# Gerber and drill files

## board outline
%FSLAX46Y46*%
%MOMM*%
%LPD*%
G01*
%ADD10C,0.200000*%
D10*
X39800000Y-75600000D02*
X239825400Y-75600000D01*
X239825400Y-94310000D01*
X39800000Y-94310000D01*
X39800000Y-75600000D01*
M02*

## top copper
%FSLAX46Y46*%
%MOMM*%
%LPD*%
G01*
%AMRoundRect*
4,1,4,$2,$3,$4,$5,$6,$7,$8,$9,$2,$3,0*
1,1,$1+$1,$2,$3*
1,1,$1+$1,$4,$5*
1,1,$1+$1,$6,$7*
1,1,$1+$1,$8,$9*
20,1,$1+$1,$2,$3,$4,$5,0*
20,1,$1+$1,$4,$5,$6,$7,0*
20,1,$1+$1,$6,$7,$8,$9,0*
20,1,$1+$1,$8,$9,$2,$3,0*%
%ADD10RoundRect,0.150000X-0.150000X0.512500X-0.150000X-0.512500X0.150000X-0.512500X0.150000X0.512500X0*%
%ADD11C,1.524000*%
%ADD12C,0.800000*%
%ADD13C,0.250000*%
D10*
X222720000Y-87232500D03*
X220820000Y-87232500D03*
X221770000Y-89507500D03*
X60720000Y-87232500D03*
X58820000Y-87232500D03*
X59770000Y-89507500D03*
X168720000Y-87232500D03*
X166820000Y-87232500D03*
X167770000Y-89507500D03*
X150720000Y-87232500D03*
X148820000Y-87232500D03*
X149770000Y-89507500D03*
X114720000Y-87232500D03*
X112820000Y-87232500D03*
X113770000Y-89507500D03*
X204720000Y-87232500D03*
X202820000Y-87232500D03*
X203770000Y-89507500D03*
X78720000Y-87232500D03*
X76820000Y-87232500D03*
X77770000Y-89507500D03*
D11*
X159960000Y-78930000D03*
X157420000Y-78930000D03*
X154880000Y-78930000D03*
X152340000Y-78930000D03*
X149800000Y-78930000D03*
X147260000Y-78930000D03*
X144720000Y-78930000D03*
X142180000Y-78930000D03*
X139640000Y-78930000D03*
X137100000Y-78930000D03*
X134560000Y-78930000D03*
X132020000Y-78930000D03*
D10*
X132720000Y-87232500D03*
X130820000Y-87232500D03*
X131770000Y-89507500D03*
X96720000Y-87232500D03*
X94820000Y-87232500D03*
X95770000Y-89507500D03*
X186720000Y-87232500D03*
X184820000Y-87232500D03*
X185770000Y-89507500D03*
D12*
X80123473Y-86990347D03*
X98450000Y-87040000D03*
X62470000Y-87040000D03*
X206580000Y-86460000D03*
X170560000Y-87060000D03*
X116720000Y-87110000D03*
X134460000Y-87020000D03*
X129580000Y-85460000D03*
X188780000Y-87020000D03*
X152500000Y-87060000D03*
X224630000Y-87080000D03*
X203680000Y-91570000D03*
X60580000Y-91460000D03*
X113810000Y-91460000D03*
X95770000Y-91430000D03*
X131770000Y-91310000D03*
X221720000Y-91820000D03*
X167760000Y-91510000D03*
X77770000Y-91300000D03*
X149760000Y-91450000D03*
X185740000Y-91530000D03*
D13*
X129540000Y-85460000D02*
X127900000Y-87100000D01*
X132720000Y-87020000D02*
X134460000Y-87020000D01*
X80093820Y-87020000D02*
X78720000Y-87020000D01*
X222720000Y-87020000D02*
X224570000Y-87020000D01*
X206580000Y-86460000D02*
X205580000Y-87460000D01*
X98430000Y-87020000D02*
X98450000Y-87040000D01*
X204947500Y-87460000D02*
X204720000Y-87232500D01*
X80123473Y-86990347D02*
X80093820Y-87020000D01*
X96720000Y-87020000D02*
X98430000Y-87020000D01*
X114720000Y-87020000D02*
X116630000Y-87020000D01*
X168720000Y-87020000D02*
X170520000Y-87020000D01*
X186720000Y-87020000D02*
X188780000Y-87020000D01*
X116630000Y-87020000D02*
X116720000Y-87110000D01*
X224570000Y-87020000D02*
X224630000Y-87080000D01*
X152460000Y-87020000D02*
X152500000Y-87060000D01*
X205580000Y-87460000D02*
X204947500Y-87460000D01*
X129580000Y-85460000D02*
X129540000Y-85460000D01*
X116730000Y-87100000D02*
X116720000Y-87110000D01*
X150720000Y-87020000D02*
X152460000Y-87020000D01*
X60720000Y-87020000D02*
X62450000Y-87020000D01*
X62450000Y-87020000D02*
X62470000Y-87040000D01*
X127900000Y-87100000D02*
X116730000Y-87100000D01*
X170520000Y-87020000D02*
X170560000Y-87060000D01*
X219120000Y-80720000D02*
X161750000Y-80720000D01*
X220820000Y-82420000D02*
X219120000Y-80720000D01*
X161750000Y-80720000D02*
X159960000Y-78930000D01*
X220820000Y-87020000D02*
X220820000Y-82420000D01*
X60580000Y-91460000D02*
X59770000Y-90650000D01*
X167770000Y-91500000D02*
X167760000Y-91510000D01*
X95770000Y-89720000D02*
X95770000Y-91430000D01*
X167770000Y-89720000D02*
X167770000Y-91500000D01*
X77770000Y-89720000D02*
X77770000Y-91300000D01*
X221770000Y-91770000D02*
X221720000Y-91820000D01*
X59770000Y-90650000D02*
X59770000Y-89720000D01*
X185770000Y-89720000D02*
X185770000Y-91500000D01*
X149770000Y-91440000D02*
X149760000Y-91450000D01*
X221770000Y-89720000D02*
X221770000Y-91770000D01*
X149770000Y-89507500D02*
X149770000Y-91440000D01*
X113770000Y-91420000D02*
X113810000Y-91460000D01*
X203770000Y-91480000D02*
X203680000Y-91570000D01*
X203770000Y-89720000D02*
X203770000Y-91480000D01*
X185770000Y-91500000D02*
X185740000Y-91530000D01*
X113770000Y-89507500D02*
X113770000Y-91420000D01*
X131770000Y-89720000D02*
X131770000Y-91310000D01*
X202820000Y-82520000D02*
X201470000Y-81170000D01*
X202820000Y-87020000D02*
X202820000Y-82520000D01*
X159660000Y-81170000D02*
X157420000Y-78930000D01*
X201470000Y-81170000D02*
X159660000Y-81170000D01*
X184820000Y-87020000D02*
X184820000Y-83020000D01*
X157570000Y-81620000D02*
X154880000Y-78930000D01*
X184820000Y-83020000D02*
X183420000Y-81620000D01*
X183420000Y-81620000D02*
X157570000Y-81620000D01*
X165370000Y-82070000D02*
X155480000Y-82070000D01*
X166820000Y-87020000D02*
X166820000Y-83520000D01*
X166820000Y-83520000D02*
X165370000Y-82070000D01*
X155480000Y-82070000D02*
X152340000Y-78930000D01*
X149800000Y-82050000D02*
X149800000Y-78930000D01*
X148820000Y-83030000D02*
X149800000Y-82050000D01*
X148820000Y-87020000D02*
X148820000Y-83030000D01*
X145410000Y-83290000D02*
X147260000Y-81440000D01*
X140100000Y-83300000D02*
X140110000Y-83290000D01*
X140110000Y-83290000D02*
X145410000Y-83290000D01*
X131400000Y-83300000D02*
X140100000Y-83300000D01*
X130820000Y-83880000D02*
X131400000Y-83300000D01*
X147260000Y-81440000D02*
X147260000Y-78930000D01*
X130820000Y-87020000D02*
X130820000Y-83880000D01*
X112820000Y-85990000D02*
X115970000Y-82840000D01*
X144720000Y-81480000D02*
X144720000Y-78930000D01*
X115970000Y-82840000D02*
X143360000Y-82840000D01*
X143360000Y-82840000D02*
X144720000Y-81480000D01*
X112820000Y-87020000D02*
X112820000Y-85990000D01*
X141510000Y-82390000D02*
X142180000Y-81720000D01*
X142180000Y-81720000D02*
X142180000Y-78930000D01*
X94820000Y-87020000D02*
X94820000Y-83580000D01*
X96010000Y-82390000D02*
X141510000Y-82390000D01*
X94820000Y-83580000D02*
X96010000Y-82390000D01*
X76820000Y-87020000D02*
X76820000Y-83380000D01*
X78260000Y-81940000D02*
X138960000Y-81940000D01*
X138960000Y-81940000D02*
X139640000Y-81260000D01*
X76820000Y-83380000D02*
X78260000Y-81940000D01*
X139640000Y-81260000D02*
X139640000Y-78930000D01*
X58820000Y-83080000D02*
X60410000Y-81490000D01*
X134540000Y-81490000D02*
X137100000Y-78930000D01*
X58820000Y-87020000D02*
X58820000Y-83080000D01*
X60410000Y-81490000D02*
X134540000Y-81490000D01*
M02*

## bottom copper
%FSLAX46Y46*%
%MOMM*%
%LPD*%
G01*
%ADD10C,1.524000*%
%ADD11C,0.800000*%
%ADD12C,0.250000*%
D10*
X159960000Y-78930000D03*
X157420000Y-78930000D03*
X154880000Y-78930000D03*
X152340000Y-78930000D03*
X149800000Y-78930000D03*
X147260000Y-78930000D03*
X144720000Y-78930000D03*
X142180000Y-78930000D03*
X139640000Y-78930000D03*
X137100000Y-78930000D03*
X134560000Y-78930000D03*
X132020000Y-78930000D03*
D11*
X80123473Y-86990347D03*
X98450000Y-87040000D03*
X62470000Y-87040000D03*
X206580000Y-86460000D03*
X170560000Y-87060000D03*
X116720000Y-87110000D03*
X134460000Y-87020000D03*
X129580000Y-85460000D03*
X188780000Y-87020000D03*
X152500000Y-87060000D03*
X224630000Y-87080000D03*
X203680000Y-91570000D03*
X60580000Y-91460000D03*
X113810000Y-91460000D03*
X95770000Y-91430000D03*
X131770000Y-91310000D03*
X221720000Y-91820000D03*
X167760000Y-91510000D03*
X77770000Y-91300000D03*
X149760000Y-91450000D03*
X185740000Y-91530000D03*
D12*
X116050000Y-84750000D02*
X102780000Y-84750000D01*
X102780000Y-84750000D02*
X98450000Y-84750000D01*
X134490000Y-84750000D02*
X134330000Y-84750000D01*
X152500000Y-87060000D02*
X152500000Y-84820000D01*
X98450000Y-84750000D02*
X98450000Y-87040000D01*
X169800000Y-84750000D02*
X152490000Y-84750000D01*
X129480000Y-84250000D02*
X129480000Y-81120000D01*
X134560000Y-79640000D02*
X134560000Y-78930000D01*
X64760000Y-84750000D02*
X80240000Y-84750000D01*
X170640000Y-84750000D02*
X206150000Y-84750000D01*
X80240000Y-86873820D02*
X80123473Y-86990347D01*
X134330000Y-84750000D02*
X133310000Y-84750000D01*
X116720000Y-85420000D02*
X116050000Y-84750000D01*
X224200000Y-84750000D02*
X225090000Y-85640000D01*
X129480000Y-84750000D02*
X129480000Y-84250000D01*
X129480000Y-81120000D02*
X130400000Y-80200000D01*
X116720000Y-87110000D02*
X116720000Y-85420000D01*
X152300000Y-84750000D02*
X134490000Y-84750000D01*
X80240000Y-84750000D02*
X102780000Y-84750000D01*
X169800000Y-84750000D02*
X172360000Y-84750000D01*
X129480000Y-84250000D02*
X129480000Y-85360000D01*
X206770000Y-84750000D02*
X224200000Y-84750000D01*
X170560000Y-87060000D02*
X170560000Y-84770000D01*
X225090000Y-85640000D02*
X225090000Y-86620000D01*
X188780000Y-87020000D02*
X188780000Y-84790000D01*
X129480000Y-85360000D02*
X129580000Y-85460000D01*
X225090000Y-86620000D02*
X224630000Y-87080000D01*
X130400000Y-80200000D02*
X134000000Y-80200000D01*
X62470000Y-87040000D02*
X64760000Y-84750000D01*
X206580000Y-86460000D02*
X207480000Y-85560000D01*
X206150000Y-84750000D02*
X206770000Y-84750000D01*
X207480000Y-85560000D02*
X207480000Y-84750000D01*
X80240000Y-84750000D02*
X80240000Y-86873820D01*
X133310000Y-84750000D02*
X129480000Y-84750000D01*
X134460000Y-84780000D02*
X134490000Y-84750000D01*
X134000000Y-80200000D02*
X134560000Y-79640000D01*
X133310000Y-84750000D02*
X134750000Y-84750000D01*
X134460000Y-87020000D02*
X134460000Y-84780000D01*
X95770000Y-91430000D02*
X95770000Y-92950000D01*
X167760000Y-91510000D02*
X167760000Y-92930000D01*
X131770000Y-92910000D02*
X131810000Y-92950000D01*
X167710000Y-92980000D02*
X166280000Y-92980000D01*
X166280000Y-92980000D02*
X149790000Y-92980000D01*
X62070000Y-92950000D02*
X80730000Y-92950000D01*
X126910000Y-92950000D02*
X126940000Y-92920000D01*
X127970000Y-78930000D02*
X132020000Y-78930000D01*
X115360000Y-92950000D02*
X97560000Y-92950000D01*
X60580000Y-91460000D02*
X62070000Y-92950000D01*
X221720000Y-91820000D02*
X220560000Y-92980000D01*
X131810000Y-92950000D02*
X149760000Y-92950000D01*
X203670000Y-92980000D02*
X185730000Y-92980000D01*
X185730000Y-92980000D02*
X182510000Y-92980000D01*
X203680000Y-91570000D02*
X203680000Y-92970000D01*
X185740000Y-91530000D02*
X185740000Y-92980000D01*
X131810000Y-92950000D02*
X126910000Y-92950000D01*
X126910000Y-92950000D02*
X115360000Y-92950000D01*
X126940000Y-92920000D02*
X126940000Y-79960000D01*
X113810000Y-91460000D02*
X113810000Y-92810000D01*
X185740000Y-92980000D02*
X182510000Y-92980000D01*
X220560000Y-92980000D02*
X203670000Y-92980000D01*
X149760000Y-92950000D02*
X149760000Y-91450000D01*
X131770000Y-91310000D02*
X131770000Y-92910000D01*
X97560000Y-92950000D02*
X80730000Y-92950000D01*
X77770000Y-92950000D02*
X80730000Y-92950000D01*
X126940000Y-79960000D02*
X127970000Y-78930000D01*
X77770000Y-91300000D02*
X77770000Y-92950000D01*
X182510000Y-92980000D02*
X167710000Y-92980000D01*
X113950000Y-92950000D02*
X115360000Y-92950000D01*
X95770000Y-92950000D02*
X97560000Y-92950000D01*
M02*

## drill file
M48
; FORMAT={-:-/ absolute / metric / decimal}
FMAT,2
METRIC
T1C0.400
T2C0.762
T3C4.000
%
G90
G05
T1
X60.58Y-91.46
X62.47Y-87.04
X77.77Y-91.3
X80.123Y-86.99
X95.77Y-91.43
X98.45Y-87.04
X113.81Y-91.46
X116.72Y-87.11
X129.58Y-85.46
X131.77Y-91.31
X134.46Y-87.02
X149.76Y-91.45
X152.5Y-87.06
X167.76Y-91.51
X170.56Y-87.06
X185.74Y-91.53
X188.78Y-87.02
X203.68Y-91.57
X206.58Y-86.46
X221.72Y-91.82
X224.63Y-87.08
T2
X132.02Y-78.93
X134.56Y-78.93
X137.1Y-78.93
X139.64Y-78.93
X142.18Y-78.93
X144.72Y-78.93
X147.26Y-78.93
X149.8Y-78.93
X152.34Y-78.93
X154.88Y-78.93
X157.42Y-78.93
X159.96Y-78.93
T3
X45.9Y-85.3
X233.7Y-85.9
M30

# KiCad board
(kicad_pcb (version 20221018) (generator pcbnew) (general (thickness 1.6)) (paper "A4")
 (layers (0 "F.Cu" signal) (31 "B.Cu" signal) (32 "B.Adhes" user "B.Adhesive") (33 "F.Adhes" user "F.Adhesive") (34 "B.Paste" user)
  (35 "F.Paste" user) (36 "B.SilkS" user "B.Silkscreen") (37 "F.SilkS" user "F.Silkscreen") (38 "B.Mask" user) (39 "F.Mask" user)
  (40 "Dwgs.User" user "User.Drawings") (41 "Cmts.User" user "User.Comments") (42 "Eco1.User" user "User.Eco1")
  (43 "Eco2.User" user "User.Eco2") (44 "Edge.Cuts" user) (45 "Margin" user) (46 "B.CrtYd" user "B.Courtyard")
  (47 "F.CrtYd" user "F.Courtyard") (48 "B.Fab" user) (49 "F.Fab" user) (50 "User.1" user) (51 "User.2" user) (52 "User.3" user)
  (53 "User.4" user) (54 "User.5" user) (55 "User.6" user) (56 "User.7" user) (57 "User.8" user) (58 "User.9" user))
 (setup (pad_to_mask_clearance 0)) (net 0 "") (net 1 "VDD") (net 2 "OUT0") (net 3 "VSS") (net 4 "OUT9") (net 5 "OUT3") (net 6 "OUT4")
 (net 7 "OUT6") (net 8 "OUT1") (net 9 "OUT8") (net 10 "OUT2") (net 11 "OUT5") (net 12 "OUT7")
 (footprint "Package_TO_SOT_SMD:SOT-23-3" (layer "F.Cu") (at 221.77 88.37 -90)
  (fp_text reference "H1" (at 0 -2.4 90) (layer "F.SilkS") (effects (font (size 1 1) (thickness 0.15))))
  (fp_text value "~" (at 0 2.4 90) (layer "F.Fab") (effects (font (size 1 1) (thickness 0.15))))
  (pad "1" smd roundrect (at -1.1375 -0.95 270) (size 1.325 0.6) (layers "F.Cu" "F.Paste" "F.Mask") (roundrect_rratio 0.25) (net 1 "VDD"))
  (pad "2" smd roundrect (at -1.1375 0.95 270) (size 1.325 0.6) (layers "F.Cu" "F.Paste" "F.Mask") (roundrect_rratio 0.25) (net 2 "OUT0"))
  (pad "3" smd roundrect (at 1.1375 0 270) (size 1.325 0.6) (layers "F.Cu" "F.Paste" "F.Mask") (roundrect_rratio 0.25) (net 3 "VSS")))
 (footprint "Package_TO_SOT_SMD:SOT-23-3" (layer "F.Cu") (at 59.77 88.37 -90)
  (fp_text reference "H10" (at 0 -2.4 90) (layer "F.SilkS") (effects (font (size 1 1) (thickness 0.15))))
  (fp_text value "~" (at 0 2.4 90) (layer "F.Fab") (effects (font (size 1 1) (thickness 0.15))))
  (pad "1" smd roundrect (at -1.1375 -0.95 270) (size 1.325 0.6) (layers "F.Cu" "F.Paste" "F.Mask") (roundrect_rratio 0.25) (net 1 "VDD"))
  (pad "2" smd roundrect (at -1.1375 0.95 270) (size 1.325 0.6) (layers "F.Cu" "F.Paste" "F.Mask") (roundrect_rratio 0.25) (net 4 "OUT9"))
  (pad "3" smd roundrect (at 1.1375 0 270) (size 1.325 0.6) (layers "F.Cu" "F.Paste" "F.Mask") (roundrect_rratio 0.25) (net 3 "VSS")))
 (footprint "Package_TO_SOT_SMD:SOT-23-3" (layer "F.Cu") (at 167.77 88.37 -90)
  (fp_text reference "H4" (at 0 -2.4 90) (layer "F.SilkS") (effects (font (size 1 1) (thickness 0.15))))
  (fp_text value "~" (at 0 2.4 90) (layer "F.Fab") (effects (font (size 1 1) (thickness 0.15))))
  (pad "1" smd roundrect (at -1.1375 -0.95 270) (size 1.325 0.6) (layers "F.Cu" "F.Paste" "F.Mask") (roundrect_rratio 0.25) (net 1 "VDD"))
  (pad "2" smd roundrect (at -1.1375 0.95 270) (size 1.325 0.6) (layers "F.Cu" "F.Paste" "F.Mask") (roundrect_rratio 0.25) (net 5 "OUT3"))
  (pad "3" smd roundrect (at 1.1375 0 270) (size 1.325 0.6) (layers "F.Cu" "F.Paste" "F.Mask") (roundrect_rratio 0.25) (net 3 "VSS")))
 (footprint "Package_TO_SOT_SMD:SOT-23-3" (layer "F.Cu") (at 149.77 88.37 -90)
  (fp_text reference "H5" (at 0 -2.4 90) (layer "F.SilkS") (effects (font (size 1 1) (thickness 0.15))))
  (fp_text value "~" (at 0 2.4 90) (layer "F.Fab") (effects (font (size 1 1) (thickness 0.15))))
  (pad "1" smd roundrect (at -1.1375 -0.95 270) (size 1.325 0.6) (layers "F.Cu" "F.Paste" "F.Mask") (roundrect_rratio 0.25) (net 1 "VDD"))
  (pad "2" smd roundrect (at -1.1375 0.95 270) (size 1.325 0.6) (layers "F.Cu" "F.Paste" "F.Mask") (roundrect_rratio 0.25) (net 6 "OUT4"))
  (pad "3" smd roundrect (at 1.1375 0 270) (size 1.325 0.6) (layers "F.Cu" "F.Paste" "F.Mask") (roundrect_rratio 0.25) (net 3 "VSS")))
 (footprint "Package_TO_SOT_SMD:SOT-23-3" (layer "F.Cu") (at 113.77 88.37 -90)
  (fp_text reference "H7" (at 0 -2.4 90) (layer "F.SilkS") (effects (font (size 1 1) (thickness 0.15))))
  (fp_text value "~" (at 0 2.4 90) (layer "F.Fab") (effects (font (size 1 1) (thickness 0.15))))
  (pad "1" smd roundrect (at -1.1375 -0.95 270) (size 1.325 0.6) (layers "F.Cu" "F.Paste" "F.Mask") (roundrect_rratio 0.25) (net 1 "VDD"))
  (pad "2" smd roundrect (at -1.1375 0.95 270) (size 1.325 0.6) (layers "F.Cu" "F.Paste" "F.Mask") (roundrect_rratio 0.25) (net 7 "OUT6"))
  (pad "3" smd roundrect (at 1.1375 0 270) (size 1.325 0.6) (layers "F.Cu" "F.Paste" "F.Mask") (roundrect_rratio 0.25) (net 3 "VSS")))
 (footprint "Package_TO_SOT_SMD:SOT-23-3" (layer "F.Cu") (at 203.77 88.37 -90)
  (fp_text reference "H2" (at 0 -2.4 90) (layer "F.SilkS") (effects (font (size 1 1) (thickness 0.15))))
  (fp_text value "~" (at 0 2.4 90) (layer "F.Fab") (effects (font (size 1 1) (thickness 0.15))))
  (pad "1" smd roundrect (at -1.1375 -0.95 270) (size 1.325 0.6) (layers "F.Cu" "F.Paste" "F.Mask") (roundrect_rratio 0.25) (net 1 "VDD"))
  (pad "2" smd roundrect (at -1.1375 0.95 270) (size 1.325 0.6) (layers "F.Cu" "F.Paste" "F.Mask") (roundrect_rratio 0.25) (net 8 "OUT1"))
  (pad "3" smd roundrect (at 1.1375 0 270) (size 1.325 0.6) (layers "F.Cu" "F.Paste" "F.Mask") (roundrect_rratio 0.25) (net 3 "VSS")))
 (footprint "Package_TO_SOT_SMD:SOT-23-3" (layer "F.Cu") (at 77.77 88.37 -90)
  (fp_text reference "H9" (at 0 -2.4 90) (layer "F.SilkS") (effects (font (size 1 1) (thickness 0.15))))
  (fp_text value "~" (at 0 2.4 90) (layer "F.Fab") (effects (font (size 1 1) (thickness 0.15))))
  (pad "1" smd roundrect (at -1.1375 -0.95 270) (size 1.325 0.6) (layers "F.Cu" "F.Paste" "F.Mask") (roundrect_rratio 0.25) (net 1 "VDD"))
  (pad "2" smd roundrect (at -1.1375 0.95 270) (size 1.325 0.6) (layers "F.Cu" "F.Paste" "F.Mask") (roundrect_rratio 0.25) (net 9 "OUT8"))
  (pad "3" smd roundrect (at 1.1375 0 270) (size 1.325 0.6) (layers "F.Cu" "F.Paste" "F.Mask") (roundrect_rratio 0.25) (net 3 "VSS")))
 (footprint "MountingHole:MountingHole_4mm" (layer "F.Cu") (at 233.7 85.9)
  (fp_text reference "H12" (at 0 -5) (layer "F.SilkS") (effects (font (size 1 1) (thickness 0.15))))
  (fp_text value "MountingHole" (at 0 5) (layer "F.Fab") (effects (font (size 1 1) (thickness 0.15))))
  (pad "" np_thru_hole circle (at 0 0) (size 4 4) (drill 4) (layers "*.Cu" "*.Mask")))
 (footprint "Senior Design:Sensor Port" (layer "F.Cu") (at 142.18 86.55 180)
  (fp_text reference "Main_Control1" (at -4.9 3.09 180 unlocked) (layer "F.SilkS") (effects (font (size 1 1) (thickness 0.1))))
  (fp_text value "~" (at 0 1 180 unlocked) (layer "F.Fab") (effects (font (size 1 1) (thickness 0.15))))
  (pad "1" thru_hole circle (at -17.78 7.62 180) (size 1.524 1.524) (drill 0.762) (layers "*.Cu" "*.Mask") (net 2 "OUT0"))
  (pad "2" thru_hole circle (at -15.24 7.62 180) (size 1.524 1.524) (drill 0.762) (layers "*.Cu" "*.Mask") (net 8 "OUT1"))
  (pad "3" thru_hole circle (at -12.7 7.62 180) (size 1.524 1.524) (drill 0.762) (layers "*.Cu" "*.Mask") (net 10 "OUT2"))
  (pad "4" thru_hole circle (at -10.16 7.62 180) (size 1.524 1.524) (drill 0.762) (layers "*.Cu" "*.Mask") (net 5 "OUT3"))
  (pad "5" thru_hole circle (at -7.62 7.62 180) (size 1.524 1.524) (drill 0.762) (layers "*.Cu" "*.Mask") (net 6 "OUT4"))
  (pad "6" thru_hole circle (at -5.08 7.62 180) (size 1.524 1.524) (drill 0.762) (layers "*.Cu" "*.Mask") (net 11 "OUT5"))
  (pad "7" thru_hole circle (at -2.54 7.62 180) (size 1.524 1.524) (drill 0.762) (layers "*.Cu" "*.Mask") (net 7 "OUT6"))
  (pad "8" thru_hole circle (at 0 7.62 180) (size 1.524 1.524) (drill 0.762) (layers "*.Cu" "*.Mask") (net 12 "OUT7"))
  (pad "9" thru_hole circle (at 2.54 7.62 180) (size 1.524 1.524) (drill 0.762) (layers "*.Cu" "*.Mask") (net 9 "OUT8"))
  (pad "10" thru_hole circle (at 5.08 7.62 180) (size 1.524 1.524) (drill 0.762) (layers "*.Cu" "*.Mask") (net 4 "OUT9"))
  (pad "11" thru_hole circle (at 7.62 7.62 180) (size 1.524 1.524) (drill 0.762) (layers "*.Cu" "*.Mask") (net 1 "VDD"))
  (pad "12" thru_hole circle (at 10.16 7.62 180) (size 1.524 1.524) (drill 0.762) (layers "*.Cu" "*.Mask") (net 3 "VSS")))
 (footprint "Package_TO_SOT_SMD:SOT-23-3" (layer "F.Cu") (at 131.77 88.37 -90)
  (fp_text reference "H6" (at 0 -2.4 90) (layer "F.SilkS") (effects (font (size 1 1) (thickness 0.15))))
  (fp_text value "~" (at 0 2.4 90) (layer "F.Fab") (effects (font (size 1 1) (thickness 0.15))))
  (pad "1" smd roundrect (at -1.1375 -0.95 270) (size 1.325 0.6) (layers "F.Cu" "F.Paste" "F.Mask") (roundrect_rratio 0.25) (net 1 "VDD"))
  (pad "2" smd roundrect (at -1.1375 0.95 270) (size 1.325 0.6) (layers "F.Cu" "F.Paste" "F.Mask") (roundrect_rratio 0.25) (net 11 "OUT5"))
  (pad "3" smd roundrect (at 1.1375 0 270) (size 1.325 0.6) (layers "F.Cu" "F.Paste" "F.Mask") (roundrect_rratio 0.25) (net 3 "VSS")))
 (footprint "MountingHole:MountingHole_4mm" (layer "F.Cu") (at 45.9 85.3)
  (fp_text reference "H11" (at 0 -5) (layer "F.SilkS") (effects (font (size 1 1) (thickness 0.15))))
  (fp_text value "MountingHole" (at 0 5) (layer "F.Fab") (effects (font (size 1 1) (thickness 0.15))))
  (pad "" np_thru_hole circle (at 0 0) (size 4 4) (drill 4) (layers "*.Cu" "*.Mask")))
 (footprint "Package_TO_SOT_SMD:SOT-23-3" (layer "F.Cu") (at 95.77 88.37 -90)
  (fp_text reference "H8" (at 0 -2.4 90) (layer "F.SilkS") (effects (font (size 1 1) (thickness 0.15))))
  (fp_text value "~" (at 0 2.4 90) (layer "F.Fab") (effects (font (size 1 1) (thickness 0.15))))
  (pad "1" smd roundrect (at -1.1375 -0.95 270) (size 1.325 0.6) (layers "F.Cu" "F.Paste" "F.Mask") (roundrect_rratio 0.25) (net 1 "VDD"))
  (pad "2" smd roundrect (at -1.1375 0.95 270) (size 1.325 0.6) (layers "F.Cu" "F.Paste" "F.Mask") (roundrect_rratio 0.25) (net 12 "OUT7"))
  (pad "3" smd roundrect (at 1.1375 0 270) (size 1.325 0.6) (layers "F.Cu" "F.Paste" "F.Mask") (roundrect_rratio 0.25) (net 3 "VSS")))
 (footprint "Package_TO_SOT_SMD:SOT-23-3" (layer "F.Cu") (at 185.77 88.37 -90)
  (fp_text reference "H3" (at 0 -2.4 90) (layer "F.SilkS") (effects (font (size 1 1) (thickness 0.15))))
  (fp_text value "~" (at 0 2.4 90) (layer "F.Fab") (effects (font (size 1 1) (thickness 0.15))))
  (pad "1" smd roundrect (at -1.1375 -0.95 270) (size 1.325 0.6) (layers "F.Cu" "F.Paste" "F.Mask") (roundrect_rratio 0.25) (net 1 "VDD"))
  (pad "2" smd roundrect (at -1.1375 0.95 270) (size 1.325 0.6) (layers "F.Cu" "F.Paste" "F.Mask") (roundrect_rratio 0.25) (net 10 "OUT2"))
  (pad "3" smd roundrect (at 1.1375 0 270) (size 1.325 0.6) (layers "F.Cu" "F.Paste" "F.Mask") (roundrect_rratio 0.25) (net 3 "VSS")))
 (gr_rect (start 39.8 75.6) (end 239.8254 94.31) (stroke (width 0.2) (type default)) (fill none) (layer "Edge.Cuts"))
 (segment (start 129.54 85.46) (end 127.9 87.1) (width 0.25) (layer "F.Cu") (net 1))
 (segment (start 132.72 87.02) (end 134.46 87.02) (width 0.25) (layer "F.Cu") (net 1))
 (segment (start 80.09382 87.02) (end 78.72 87.02) (width 0.25) (layer "F.Cu") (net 1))
 (segment (start 222.72 87.02) (end 224.57 87.02) (width 0.25) (layer "F.Cu") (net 1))
 (segment (start 206.58 86.46) (end 205.58 87.46) (width 0.25) (layer "F.Cu") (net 1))
 (segment (start 98.43 87.02) (end 98.45 87.04) (width 0.25) (layer "F.Cu") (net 1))
 (segment (start 204.9475 87.46) (end 204.72 87.2325) (width 0.25) (layer "F.Cu") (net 1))
 (segment (start 80.123473 86.990347) (end 80.09382 87.02) (width 0.25) (layer "F.Cu") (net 1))
 (segment (start 96.72 87.02) (end 98.43 87.02) (width 0.25) (layer "F.Cu") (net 1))
 (segment (start 114.72 87.02) (end 116.63 87.02) (width 0.25) (layer "F.Cu") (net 1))
 (segment (start 168.72 87.02) (end 170.52 87.02) (width 0.25) (layer "F.Cu") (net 1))
 (segment (start 186.72 87.02) (end 188.78 87.02) (width 0.25) (layer "F.Cu") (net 1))
 (segment (start 116.63 87.02) (end 116.72 87.11) (width 0.25) (layer "F.Cu") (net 1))
 (segment (start 224.57 87.02) (end 224.63 87.08) (width 0.25) (layer "F.Cu") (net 1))
 (segment (start 152.46 87.02) (end 152.5 87.06) (width 0.25) (layer "F.Cu") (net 1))
 (segment (start 205.58 87.46) (end 204.9475 87.46) (width 0.25) (layer "F.Cu") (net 1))
 (segment (start 129.58 85.46) (end 129.54 85.46) (width 0.25) (layer "F.Cu") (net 1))
 (segment (start 116.73 87.1) (end 116.72 87.11) (width 0.25) (layer "F.Cu") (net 1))
 (segment (start 150.72 87.02) (end 152.46 87.02) (width 0.25) (layer "F.Cu") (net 1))
 (segment (start 60.72 87.02) (end 62.45 87.02) (width 0.25) (layer "F.Cu") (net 1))
 (segment (start 62.45 87.02) (end 62.47 87.04) (width 0.25) (layer "F.Cu") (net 1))
 (segment (start 127.9 87.1) (end 116.73 87.1) (width 0.25) (layer "F.Cu") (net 1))
 (segment (start 170.52 87.02) (end 170.56 87.06) (width 0.25) (layer "F.Cu") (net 1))
 (via (at 80.123473 86.990347) (size 0.8) (drill 0.4) (layers "F.Cu" "B.Cu") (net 1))
 (via (at 98.45 87.04) (size 0.8) (drill 0.4) (layers "F.Cu" "B.Cu") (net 1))
 (via (at 62.47 87.04) (size 0.8) (drill 0.4) (layers "F.Cu" "B.Cu") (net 1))
 (via (at 206.58 86.46) (size 0.8) (drill 0.4) (layers "F.Cu" "B.Cu") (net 1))
 (via (at 170.56 87.06) (size 0.8) (drill 0.4) (layers "F.Cu" "B.Cu") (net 1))
 (via (at 116.72 87.11) (size 0.8) (drill 0.4) (layers "F.Cu" "B.Cu") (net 1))
 (via (at 134.46 87.02) (size 0.8) (drill 0.4) (layers "F.Cu" "B.Cu") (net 1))
 (via (at 129.58 85.46) (size 0.8) (drill 0.4) (layers "F.Cu" "B.Cu") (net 1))
 (via (at 188.78 87.02) (size 0.8) (drill 0.4) (layers "F.Cu" "B.Cu") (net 1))
 (via (at 152.5 87.06) (size 0.8) (drill 0.4) (layers "F.Cu" "B.Cu") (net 1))
 (via (at 224.63 87.08) (size 0.8) (drill 0.4) (layers "F.Cu" "B.Cu") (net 1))
 (segment (start 116.05 84.75) (end 102.78 84.75) (width 0.25) (layer "B.Cu") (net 1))
 (segment (start 102.78 84.75) (end 98.45 84.75) (width 0.25) (layer "B.Cu") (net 1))
 (segment (start 134.49 84.75) (end 134.33 84.75) (width 0.25) (layer "B.Cu") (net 1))
 (segment (start 152.5 87.06) (end 152.5 84.82) (width 0.25) (layer "B.Cu") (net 1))
 (segment (start 98.45 84.75) (end 98.45 87.04) (width 0.25) (layer "B.Cu") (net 1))
 (segment (start 169.8 84.75) (end 152.49 84.75) (width 0.25) (layer "B.Cu") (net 1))
 (segment (start 129.48 84.25) (end 129.48 81.12) (width 0.25) (layer "B.Cu") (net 1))
 (segment (start 134.56 79.64) (end 134.56 78.93) (width 0.25) (layer "B.Cu") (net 1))
 (segment (start 64.76 84.75) (end 80.24 84.75) (width 0.25) (layer "B.Cu") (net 1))
 (segment (start 170.64 84.75) (end 206.15 84.75) (width 0.25) (layer "B.Cu") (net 1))
 (segment (start 80.24 86.87382) (end 80.123473 86.990347) (width 0.25) (layer "B.Cu") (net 1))
 (segment (start 134.33 84.75) (end 133.31 84.75) (width 0.25) (layer "B.Cu") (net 1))
 (segment (start 116.72 85.42) (end 116.05 84.75) (width 0.25) (layer "B.Cu") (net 1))
 (segment (start 224.2 84.75) (end 225.09 85.64) (width 0.25) (layer "B.Cu") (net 1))
 (segment (start 129.48 84.75) (end 129.48 84.25) (width 0.25) (layer "B.Cu") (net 1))
 (segment (start 129.48 81.12) (end 130.4 80.2) (width 0.25) (layer "B.Cu") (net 1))
 (segment (start 116.72 87.11) (end 116.72 85.42) (width 0.25) (layer "B.Cu") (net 1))
 (segment (start 152.3 84.75) (end 134.49 84.75) (width 0.25) (layer "B.Cu") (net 1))
 (segment (start 80.24 84.75) (end 102.78 84.75) (width 0.25) (layer "B.Cu") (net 1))
 (segment (start 169.8 84.75) (end 172.36 84.75) (width 0.25) (layer "B.Cu") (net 1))
 (segment (start 129.48 84.25) (end 129.48 85.36) (width 0.25) (layer "B.Cu") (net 1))
 (segment (start 206.77 84.75) (end 224.2 84.75) (width 0.25) (layer "B.Cu") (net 1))
 (segment (start 170.56 87.06) (end 170.56 84.77) (width 0.25) (layer "B.Cu") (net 1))
 (segment (start 225.09 85.64) (end 225.09 86.62) (width 0.25) (layer "B.Cu") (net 1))
 (segment (start 188.78 87.02) (end 188.78 84.79) (width 0.25) (layer "B.Cu") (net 1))
 (segment (start 129.48 85.36) (end 129.58 85.46) (width 0.25) (layer "B.Cu") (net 1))
 (segment (start 225.09 86.62) (end 224.63 87.08) (width 0.25) (layer "B.Cu") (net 1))
 (segment (start 130.4 80.2) (end 134 80.2) (width 0.25) (layer "B.Cu") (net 1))
 (segment (start 62.47 87.04) (end 64.76 84.75) (width 0.25) (layer "B.Cu") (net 1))
 (segment (start 206.58 86.46) (end 207.48 85.56) (width 0.25) (layer "B.Cu") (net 1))
 (segment (start 206.15 84.75) (end 206.77 84.75) (width 0.25) (layer "B.Cu") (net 1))
 (segment (start 207.48 85.56) (end 207.48 84.75) (width 0.25) (layer "B.Cu") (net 1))
 (segment (start 80.24 84.75) (end 80.24 86.87382) (width 0.25) (layer "B.Cu") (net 1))
 (segment (start 133.31 84.75) (end 129.48 84.75) (width 0.25) (layer "B.Cu") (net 1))
 (segment (start 134.46 84.78) (end 134.49 84.75) (width 0.25) (layer "B.Cu") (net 1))
 (segment (start 134 80.2) (end 134.56 79.64) (width 0.25) (layer "B.Cu") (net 1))
 (segment (start 133.31 84.75) (end 134.75 84.75) (width 0.25) (layer "B.Cu") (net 1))
 (segment (start 134.46 87.02) (end 134.46 84.78) (width 0.25) (layer "B.Cu") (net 1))
 (segment (start 219.12 80.72) (end 161.75 80.72) (width 0.25) (layer "F.Cu") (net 2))
 (segment (start 220.82 82.42) (end 219.12 80.72) (width 0.25) (layer "F.Cu") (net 2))
 (segment (start 161.75 80.72) (end 159.96 78.93) (width 0.25) (layer "F.Cu") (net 2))
 (segment (start 220.82 87.02) (end 220.82 82.42) (width 0.25) (layer "F.Cu") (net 2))
 (segment (start 60.58 91.46) (end 59.77 90.65) (width 0.25) (layer "F.Cu") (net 3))
 (segment (start 167.77 91.5) (end 167.76 91.51) (width 0.25) (layer "F.Cu") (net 3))
 (segment (start 95.77 89.72) (end 95.77 91.43) (width 0.25) (layer "F.Cu") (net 3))
 (segment (start 167.77 89.72) (end 167.77 91.5) (width 0.25) (layer "F.Cu") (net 3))
 (segment (start 77.77 89.72) (end 77.77 91.3) (width 0.25) (layer "F.Cu") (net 3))
 (segment (start 221.77 91.77) (end 221.72 91.82) (width 0.25) (layer "F.Cu") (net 3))
 (segment (start 59.77 90.65) (end 59.77 89.72) (width 0.25) (layer "F.Cu") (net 3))
 (segment (start 185.77 89.72) (end 185.77 91.5) (width 0.25) (layer "F.Cu") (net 3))
 (segment (start 149.77 91.44) (end 149.76 91.45) (width 0.25) (layer "F.Cu") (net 3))
 (segment (start 221.77 89.72) (end 221.77 91.77) (width 0.25) (layer "F.Cu") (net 3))
 (segment (start 149.77 89.5075) (end 149.77 91.44) (width 0.25) (layer "F.Cu") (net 3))
 (segment (start 113.77 91.42) (end 113.81 91.46) (width 0.25) (layer "F.Cu") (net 3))
 (segment (start 203.77 91.48) (end 203.68 91.57) (width 0.25) (layer "F.Cu") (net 3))
 (segment (start 203.77 89.72) (end 203.77 91.48) (width 0.25) (layer "F.Cu") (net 3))
 (segment (start 185.77 91.5) (end 185.74 91.53) (width 0.25) (layer "F.Cu") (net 3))
 (segment (start 113.77 89.5075) (end 113.77 91.42) (width 0.25) (layer "F.Cu") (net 3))
 (segment (start 131.77 89.72) (end 131.77 91.31) (width 0.25) (layer "F.Cu") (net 3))
 (via (at 203.68 91.57) (size 0.8) (drill 0.4) (layers "F.Cu" "B.Cu") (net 3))
 (via (at 60.58 91.46) (size 0.8) (drill 0.4) (layers "F.Cu" "B.Cu") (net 3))
 (via (at 113.81 91.46) (size 0.8) (drill 0.4) (layers "F.Cu" "B.Cu") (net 3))
 (via (at 95.77 91.43) (size 0.8) (drill 0.4) (layers "F.Cu" "B.Cu") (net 3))
 (via (at 131.77 91.31) (size 0.8) (drill 0.4) (layers "F.Cu" "B.Cu") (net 3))
 (via (at 221.72 91.82) (size 0.8) (drill 0.4) (layers "F.Cu" "B.Cu") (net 3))
 (via (at 167.76 91.51) (size 0.8) (drill 0.4) (layers "F.Cu" "B.Cu") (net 3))
 (via (at 77.77 91.3) (size 0.8) (drill 0.4) (layers "F.Cu" "B.Cu") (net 3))
 (via (at 149.76 91.45) (size 0.8) (drill 0.4) (layers "F.Cu" "B.Cu") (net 3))
 (via (at 185.74 91.53) (size 0.8) (drill 0.4) (layers "F.Cu" "B.Cu") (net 3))
 (segment (start 95.77 91.43) (end 95.77 92.95) (width 0.25) (layer "B.Cu") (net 3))
 (segment (start 167.76 91.51) (end 167.76 92.93) (width 0.25) (layer "B.Cu") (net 3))
 (segment (start 131.77 92.91) (end 131.81 92.95) (width 0.25) (layer "B.Cu") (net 3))
 (segment (start 167.71 92.98) (end 166.28 92.98) (width 0.25) (layer "B.Cu") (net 3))
 (segment (start 166.28 92.98) (end 149.79 92.98) (width 0.25) (layer "B.Cu") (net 3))
 (segment (start 62.07 92.95) (end 80.73 92.95) (width 0.25) (layer "B.Cu") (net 3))
 (segment (start 126.91 92.95) (end 126.94 92.92) (width 0.25) (layer "B.Cu") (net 3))
 (segment (start 127.97 78.93) (end 132.02 78.93) (width 0.25) (layer "B.Cu") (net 3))
 (segment (start 115.36 92.95) (end 97.56 92.95) (width 0.25) (layer "B.Cu") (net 3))
 (segment (start 60.58 91.46) (end 62.07 92.95) (width 0.25) (layer "B.Cu") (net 3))
 (segment (start 221.72 91.82) (end 220.56 92.98) (width 0.25) (layer "B.Cu") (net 3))
 (segment (start 131.81 92.95) (end 149.76 92.95) (width 0.25) (layer "B.Cu") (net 3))
 (segment (start 203.67 92.98) (end 185.73 92.98) (width 0.25) (layer "B.Cu") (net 3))
 (segment (start 185.73 92.98) (end 182.51 92.98) (width 0.25) (layer "B.Cu") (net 3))
 (segment (start 203.68 91.57) (end 203.68 92.97) (width 0.25) (layer "B.Cu") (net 3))
 (segment (start 185.74 91.53) (end 185.74 92.98) (width 0.25) (layer "B.Cu") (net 3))
 (segment (start 131.81 92.95) (end 126.91 92.95) (width 0.25) (layer "B.Cu") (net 3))
 (segment (start 126.91 92.95) (end 115.36 92.95) (width 0.25) (layer "B.Cu") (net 3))
 (segment (start 126.94 92.92) (end 126.94 79.96) (width 0.25) (layer "B.Cu") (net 3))
 (segment (start 113.81 91.46) (end 113.81 92.81) (width 0.25) (layer "B.Cu") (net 3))
 (segment (start 185.74 92.98) (end 182.51 92.98) (width 0.25) (layer "B.Cu") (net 3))
 (segment (start 220.56 92.98) (end 203.67 92.98) (width 0.25) (layer "B.Cu") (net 3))
 (segment (start 149.76 92.95) (end 149.76 91.45) (width 0.25) (layer "B.Cu") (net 3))
 (segment (start 131.77 91.31) (end 131.77 92.91) (width 0.25) (layer "B.Cu") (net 3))
 (segment (start 97.56 92.95) (end 80.73 92.95) (width 0.25) (layer "B.Cu") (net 3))
 (segment (start 77.77 92.95) (end 80.73 92.95) (width 0.25) (layer "B.Cu") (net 3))
 (segment (start 126.94 79.96) (end 127.97 78.93) (width 0.25) (layer "B.Cu") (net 3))
 (segment (start 77.77 91.3) (end 77.77 92.95) (width 0.25) (layer "B.Cu") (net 3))
 (segment (start 182.51 92.98) (end 167.71 92.98) (width 0.25) (layer "B.Cu") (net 3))
 (segment (start 113.95 92.95) (end 115.36 92.95) (width 0.25) (layer "B.Cu") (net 3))
 (segment (start 95.77 92.95) (end 97.56 92.95) (width 0.25) (layer "B.Cu") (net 3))
 (segment (start 202.82 82.52) (end 201.47 81.17) (width 0.25) (layer "F.Cu") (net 8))
 (segment (start 202.82 87.02) (end 202.82 82.52) (width 0.25) (layer "F.Cu") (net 8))
 (segment (start 159.66 81.17) (end 157.42 78.93) (width 0.25) (layer "F.Cu") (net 8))
 (segment (start 201.47 81.17) (end 159.66 81.17) (width 0.25) (layer "F.Cu") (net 8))
 (segment (start 184.82 87.02) (end 184.82 83.02) (width 0.25) (layer "F.Cu") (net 10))
 (segment (start 157.57 81.62) (end 154.88 78.93) (width 0.25) (layer "F.Cu") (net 10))
 (segment (start 184.82 83.02) (end 183.42 81.62) (width 0.25) (layer "F.Cu") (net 10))
 (segment (start 183.42 81.62) (end 157.57 81.62) (width 0.25) (layer "F.Cu") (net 10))
 (segment (start 165.37 82.07) (end 155.48 82.07) (width 0.25) (layer "F.Cu") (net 5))
 (segment (start 166.82 87.02) (end 166.82 83.52) (width 0.25) (layer "F.Cu") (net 5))
 (segment (start 166.82 83.52) (end 165.37 82.07) (width 0.25) (layer "F.Cu") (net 5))
 (segment (start 155.48 82.07) (end 152.34 78.93) (width 0.25) (layer "F.Cu") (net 5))
 (segment (start 149.8 82.05) (end 149.8 78.93) (width 0.25) (layer "F.Cu") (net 6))
 (segment (start 148.82 83.03) (end 149.8 82.05) (width 0.25) (layer "F.Cu") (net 6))
 (segment (start 148.82 87.02) (end 148.82 83.03) (width 0.25) (layer "F.Cu") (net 6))
 (segment (start 145.41 83.29) (end 147.26 81.44) (width 0.25) (layer "F.Cu") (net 11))
 (segment (start 140.1 83.3) (end 140.11 83.29) (width 0.25) (layer "F.Cu") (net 11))
 (segment (start 140.11 83.29) (end 145.41 83.29) (width 0.25) (layer "F.Cu") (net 11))
 (segment (start 131.4 83.3) (end 140.1 83.3) (width 0.25) (layer "F.Cu") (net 11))
 (segment (start 130.82 83.88) (end 131.4 83.3) (width 0.25) (layer "F.Cu") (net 11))
 (segment (start 147.26 81.44) (end 147.26 78.93) (width 0.25) (layer "F.Cu") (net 11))
 (segment (start 130.82 87.02) (end 130.82 83.88) (width 0.25) (layer "F.Cu") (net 11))
 (segment (start 112.82 85.99) (end 115.97 82.84) (width 0.25) (layer "F.Cu") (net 7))
 (segment (start 144.72 81.48) (end 144.72 78.93) (width 0.25) (layer "F.Cu") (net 7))
 (segment (start 115.97 82.84) (end 143.36 82.84) (width 0.25) (layer "F.Cu") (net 7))
 (segment (start 143.36 82.84) (end 144.72 81.48) (width 0.25) (layer "F.Cu") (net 7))
 (segment (start 112.82 87.02) (end 112.82 85.99) (width 0.25) (layer "F.Cu") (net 7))
 (segment (start 141.51 82.39) (end 142.18 81.72) (width 0.25) (layer "F.Cu") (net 12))
 (segment (start 142.18 81.72) (end 142.18 78.93) (width 0.25) (layer "F.Cu") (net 12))
 (segment (start 94.82 87.02) (end 94.82 83.58) (width 0.25) (layer "F.Cu") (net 12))
 (segment (start 96.01 82.39) (end 141.51 82.39) (width 0.25) (layer "F.Cu") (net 12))
 (segment (start 94.82 83.58) (end 96.01 82.39) (width 0.25) (layer "F.Cu") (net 12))
 (segment (start 76.82 87.02) (end 76.82 83.38) (width 0.25) (layer "F.Cu") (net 9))
 (segment (start 78.26 81.94) (end 138.96 81.94) (width 0.25) (layer "F.Cu") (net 9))
 (segment (start 138.96 81.94) (end 139.64 81.26) (width 0.25) (layer "F.Cu") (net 9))
 (segment (start 76.82 83.38) (end 78.26 81.94) (width 0.25) (layer "F.Cu") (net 9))
 (segment (start 139.64 81.26) (end 139.64 78.93) (width 0.25) (layer "F.Cu") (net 9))
 (segment (start 58.82 83.08) (end 60.41 81.49) (width 0.25) (layer "F.Cu") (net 4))
 (segment (start 134.54 81.49) (end 137.1 78.93) (width 0.25) (layer "F.Cu") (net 4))
 (segment (start 58.82 87.02) (end 58.82 83.08) (width 0.25) (layer "F.Cu") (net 4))
 (segment (start 60.41 81.49) (end 134.54 81.49) (width 0.25) (layer "F.Cu") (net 4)))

